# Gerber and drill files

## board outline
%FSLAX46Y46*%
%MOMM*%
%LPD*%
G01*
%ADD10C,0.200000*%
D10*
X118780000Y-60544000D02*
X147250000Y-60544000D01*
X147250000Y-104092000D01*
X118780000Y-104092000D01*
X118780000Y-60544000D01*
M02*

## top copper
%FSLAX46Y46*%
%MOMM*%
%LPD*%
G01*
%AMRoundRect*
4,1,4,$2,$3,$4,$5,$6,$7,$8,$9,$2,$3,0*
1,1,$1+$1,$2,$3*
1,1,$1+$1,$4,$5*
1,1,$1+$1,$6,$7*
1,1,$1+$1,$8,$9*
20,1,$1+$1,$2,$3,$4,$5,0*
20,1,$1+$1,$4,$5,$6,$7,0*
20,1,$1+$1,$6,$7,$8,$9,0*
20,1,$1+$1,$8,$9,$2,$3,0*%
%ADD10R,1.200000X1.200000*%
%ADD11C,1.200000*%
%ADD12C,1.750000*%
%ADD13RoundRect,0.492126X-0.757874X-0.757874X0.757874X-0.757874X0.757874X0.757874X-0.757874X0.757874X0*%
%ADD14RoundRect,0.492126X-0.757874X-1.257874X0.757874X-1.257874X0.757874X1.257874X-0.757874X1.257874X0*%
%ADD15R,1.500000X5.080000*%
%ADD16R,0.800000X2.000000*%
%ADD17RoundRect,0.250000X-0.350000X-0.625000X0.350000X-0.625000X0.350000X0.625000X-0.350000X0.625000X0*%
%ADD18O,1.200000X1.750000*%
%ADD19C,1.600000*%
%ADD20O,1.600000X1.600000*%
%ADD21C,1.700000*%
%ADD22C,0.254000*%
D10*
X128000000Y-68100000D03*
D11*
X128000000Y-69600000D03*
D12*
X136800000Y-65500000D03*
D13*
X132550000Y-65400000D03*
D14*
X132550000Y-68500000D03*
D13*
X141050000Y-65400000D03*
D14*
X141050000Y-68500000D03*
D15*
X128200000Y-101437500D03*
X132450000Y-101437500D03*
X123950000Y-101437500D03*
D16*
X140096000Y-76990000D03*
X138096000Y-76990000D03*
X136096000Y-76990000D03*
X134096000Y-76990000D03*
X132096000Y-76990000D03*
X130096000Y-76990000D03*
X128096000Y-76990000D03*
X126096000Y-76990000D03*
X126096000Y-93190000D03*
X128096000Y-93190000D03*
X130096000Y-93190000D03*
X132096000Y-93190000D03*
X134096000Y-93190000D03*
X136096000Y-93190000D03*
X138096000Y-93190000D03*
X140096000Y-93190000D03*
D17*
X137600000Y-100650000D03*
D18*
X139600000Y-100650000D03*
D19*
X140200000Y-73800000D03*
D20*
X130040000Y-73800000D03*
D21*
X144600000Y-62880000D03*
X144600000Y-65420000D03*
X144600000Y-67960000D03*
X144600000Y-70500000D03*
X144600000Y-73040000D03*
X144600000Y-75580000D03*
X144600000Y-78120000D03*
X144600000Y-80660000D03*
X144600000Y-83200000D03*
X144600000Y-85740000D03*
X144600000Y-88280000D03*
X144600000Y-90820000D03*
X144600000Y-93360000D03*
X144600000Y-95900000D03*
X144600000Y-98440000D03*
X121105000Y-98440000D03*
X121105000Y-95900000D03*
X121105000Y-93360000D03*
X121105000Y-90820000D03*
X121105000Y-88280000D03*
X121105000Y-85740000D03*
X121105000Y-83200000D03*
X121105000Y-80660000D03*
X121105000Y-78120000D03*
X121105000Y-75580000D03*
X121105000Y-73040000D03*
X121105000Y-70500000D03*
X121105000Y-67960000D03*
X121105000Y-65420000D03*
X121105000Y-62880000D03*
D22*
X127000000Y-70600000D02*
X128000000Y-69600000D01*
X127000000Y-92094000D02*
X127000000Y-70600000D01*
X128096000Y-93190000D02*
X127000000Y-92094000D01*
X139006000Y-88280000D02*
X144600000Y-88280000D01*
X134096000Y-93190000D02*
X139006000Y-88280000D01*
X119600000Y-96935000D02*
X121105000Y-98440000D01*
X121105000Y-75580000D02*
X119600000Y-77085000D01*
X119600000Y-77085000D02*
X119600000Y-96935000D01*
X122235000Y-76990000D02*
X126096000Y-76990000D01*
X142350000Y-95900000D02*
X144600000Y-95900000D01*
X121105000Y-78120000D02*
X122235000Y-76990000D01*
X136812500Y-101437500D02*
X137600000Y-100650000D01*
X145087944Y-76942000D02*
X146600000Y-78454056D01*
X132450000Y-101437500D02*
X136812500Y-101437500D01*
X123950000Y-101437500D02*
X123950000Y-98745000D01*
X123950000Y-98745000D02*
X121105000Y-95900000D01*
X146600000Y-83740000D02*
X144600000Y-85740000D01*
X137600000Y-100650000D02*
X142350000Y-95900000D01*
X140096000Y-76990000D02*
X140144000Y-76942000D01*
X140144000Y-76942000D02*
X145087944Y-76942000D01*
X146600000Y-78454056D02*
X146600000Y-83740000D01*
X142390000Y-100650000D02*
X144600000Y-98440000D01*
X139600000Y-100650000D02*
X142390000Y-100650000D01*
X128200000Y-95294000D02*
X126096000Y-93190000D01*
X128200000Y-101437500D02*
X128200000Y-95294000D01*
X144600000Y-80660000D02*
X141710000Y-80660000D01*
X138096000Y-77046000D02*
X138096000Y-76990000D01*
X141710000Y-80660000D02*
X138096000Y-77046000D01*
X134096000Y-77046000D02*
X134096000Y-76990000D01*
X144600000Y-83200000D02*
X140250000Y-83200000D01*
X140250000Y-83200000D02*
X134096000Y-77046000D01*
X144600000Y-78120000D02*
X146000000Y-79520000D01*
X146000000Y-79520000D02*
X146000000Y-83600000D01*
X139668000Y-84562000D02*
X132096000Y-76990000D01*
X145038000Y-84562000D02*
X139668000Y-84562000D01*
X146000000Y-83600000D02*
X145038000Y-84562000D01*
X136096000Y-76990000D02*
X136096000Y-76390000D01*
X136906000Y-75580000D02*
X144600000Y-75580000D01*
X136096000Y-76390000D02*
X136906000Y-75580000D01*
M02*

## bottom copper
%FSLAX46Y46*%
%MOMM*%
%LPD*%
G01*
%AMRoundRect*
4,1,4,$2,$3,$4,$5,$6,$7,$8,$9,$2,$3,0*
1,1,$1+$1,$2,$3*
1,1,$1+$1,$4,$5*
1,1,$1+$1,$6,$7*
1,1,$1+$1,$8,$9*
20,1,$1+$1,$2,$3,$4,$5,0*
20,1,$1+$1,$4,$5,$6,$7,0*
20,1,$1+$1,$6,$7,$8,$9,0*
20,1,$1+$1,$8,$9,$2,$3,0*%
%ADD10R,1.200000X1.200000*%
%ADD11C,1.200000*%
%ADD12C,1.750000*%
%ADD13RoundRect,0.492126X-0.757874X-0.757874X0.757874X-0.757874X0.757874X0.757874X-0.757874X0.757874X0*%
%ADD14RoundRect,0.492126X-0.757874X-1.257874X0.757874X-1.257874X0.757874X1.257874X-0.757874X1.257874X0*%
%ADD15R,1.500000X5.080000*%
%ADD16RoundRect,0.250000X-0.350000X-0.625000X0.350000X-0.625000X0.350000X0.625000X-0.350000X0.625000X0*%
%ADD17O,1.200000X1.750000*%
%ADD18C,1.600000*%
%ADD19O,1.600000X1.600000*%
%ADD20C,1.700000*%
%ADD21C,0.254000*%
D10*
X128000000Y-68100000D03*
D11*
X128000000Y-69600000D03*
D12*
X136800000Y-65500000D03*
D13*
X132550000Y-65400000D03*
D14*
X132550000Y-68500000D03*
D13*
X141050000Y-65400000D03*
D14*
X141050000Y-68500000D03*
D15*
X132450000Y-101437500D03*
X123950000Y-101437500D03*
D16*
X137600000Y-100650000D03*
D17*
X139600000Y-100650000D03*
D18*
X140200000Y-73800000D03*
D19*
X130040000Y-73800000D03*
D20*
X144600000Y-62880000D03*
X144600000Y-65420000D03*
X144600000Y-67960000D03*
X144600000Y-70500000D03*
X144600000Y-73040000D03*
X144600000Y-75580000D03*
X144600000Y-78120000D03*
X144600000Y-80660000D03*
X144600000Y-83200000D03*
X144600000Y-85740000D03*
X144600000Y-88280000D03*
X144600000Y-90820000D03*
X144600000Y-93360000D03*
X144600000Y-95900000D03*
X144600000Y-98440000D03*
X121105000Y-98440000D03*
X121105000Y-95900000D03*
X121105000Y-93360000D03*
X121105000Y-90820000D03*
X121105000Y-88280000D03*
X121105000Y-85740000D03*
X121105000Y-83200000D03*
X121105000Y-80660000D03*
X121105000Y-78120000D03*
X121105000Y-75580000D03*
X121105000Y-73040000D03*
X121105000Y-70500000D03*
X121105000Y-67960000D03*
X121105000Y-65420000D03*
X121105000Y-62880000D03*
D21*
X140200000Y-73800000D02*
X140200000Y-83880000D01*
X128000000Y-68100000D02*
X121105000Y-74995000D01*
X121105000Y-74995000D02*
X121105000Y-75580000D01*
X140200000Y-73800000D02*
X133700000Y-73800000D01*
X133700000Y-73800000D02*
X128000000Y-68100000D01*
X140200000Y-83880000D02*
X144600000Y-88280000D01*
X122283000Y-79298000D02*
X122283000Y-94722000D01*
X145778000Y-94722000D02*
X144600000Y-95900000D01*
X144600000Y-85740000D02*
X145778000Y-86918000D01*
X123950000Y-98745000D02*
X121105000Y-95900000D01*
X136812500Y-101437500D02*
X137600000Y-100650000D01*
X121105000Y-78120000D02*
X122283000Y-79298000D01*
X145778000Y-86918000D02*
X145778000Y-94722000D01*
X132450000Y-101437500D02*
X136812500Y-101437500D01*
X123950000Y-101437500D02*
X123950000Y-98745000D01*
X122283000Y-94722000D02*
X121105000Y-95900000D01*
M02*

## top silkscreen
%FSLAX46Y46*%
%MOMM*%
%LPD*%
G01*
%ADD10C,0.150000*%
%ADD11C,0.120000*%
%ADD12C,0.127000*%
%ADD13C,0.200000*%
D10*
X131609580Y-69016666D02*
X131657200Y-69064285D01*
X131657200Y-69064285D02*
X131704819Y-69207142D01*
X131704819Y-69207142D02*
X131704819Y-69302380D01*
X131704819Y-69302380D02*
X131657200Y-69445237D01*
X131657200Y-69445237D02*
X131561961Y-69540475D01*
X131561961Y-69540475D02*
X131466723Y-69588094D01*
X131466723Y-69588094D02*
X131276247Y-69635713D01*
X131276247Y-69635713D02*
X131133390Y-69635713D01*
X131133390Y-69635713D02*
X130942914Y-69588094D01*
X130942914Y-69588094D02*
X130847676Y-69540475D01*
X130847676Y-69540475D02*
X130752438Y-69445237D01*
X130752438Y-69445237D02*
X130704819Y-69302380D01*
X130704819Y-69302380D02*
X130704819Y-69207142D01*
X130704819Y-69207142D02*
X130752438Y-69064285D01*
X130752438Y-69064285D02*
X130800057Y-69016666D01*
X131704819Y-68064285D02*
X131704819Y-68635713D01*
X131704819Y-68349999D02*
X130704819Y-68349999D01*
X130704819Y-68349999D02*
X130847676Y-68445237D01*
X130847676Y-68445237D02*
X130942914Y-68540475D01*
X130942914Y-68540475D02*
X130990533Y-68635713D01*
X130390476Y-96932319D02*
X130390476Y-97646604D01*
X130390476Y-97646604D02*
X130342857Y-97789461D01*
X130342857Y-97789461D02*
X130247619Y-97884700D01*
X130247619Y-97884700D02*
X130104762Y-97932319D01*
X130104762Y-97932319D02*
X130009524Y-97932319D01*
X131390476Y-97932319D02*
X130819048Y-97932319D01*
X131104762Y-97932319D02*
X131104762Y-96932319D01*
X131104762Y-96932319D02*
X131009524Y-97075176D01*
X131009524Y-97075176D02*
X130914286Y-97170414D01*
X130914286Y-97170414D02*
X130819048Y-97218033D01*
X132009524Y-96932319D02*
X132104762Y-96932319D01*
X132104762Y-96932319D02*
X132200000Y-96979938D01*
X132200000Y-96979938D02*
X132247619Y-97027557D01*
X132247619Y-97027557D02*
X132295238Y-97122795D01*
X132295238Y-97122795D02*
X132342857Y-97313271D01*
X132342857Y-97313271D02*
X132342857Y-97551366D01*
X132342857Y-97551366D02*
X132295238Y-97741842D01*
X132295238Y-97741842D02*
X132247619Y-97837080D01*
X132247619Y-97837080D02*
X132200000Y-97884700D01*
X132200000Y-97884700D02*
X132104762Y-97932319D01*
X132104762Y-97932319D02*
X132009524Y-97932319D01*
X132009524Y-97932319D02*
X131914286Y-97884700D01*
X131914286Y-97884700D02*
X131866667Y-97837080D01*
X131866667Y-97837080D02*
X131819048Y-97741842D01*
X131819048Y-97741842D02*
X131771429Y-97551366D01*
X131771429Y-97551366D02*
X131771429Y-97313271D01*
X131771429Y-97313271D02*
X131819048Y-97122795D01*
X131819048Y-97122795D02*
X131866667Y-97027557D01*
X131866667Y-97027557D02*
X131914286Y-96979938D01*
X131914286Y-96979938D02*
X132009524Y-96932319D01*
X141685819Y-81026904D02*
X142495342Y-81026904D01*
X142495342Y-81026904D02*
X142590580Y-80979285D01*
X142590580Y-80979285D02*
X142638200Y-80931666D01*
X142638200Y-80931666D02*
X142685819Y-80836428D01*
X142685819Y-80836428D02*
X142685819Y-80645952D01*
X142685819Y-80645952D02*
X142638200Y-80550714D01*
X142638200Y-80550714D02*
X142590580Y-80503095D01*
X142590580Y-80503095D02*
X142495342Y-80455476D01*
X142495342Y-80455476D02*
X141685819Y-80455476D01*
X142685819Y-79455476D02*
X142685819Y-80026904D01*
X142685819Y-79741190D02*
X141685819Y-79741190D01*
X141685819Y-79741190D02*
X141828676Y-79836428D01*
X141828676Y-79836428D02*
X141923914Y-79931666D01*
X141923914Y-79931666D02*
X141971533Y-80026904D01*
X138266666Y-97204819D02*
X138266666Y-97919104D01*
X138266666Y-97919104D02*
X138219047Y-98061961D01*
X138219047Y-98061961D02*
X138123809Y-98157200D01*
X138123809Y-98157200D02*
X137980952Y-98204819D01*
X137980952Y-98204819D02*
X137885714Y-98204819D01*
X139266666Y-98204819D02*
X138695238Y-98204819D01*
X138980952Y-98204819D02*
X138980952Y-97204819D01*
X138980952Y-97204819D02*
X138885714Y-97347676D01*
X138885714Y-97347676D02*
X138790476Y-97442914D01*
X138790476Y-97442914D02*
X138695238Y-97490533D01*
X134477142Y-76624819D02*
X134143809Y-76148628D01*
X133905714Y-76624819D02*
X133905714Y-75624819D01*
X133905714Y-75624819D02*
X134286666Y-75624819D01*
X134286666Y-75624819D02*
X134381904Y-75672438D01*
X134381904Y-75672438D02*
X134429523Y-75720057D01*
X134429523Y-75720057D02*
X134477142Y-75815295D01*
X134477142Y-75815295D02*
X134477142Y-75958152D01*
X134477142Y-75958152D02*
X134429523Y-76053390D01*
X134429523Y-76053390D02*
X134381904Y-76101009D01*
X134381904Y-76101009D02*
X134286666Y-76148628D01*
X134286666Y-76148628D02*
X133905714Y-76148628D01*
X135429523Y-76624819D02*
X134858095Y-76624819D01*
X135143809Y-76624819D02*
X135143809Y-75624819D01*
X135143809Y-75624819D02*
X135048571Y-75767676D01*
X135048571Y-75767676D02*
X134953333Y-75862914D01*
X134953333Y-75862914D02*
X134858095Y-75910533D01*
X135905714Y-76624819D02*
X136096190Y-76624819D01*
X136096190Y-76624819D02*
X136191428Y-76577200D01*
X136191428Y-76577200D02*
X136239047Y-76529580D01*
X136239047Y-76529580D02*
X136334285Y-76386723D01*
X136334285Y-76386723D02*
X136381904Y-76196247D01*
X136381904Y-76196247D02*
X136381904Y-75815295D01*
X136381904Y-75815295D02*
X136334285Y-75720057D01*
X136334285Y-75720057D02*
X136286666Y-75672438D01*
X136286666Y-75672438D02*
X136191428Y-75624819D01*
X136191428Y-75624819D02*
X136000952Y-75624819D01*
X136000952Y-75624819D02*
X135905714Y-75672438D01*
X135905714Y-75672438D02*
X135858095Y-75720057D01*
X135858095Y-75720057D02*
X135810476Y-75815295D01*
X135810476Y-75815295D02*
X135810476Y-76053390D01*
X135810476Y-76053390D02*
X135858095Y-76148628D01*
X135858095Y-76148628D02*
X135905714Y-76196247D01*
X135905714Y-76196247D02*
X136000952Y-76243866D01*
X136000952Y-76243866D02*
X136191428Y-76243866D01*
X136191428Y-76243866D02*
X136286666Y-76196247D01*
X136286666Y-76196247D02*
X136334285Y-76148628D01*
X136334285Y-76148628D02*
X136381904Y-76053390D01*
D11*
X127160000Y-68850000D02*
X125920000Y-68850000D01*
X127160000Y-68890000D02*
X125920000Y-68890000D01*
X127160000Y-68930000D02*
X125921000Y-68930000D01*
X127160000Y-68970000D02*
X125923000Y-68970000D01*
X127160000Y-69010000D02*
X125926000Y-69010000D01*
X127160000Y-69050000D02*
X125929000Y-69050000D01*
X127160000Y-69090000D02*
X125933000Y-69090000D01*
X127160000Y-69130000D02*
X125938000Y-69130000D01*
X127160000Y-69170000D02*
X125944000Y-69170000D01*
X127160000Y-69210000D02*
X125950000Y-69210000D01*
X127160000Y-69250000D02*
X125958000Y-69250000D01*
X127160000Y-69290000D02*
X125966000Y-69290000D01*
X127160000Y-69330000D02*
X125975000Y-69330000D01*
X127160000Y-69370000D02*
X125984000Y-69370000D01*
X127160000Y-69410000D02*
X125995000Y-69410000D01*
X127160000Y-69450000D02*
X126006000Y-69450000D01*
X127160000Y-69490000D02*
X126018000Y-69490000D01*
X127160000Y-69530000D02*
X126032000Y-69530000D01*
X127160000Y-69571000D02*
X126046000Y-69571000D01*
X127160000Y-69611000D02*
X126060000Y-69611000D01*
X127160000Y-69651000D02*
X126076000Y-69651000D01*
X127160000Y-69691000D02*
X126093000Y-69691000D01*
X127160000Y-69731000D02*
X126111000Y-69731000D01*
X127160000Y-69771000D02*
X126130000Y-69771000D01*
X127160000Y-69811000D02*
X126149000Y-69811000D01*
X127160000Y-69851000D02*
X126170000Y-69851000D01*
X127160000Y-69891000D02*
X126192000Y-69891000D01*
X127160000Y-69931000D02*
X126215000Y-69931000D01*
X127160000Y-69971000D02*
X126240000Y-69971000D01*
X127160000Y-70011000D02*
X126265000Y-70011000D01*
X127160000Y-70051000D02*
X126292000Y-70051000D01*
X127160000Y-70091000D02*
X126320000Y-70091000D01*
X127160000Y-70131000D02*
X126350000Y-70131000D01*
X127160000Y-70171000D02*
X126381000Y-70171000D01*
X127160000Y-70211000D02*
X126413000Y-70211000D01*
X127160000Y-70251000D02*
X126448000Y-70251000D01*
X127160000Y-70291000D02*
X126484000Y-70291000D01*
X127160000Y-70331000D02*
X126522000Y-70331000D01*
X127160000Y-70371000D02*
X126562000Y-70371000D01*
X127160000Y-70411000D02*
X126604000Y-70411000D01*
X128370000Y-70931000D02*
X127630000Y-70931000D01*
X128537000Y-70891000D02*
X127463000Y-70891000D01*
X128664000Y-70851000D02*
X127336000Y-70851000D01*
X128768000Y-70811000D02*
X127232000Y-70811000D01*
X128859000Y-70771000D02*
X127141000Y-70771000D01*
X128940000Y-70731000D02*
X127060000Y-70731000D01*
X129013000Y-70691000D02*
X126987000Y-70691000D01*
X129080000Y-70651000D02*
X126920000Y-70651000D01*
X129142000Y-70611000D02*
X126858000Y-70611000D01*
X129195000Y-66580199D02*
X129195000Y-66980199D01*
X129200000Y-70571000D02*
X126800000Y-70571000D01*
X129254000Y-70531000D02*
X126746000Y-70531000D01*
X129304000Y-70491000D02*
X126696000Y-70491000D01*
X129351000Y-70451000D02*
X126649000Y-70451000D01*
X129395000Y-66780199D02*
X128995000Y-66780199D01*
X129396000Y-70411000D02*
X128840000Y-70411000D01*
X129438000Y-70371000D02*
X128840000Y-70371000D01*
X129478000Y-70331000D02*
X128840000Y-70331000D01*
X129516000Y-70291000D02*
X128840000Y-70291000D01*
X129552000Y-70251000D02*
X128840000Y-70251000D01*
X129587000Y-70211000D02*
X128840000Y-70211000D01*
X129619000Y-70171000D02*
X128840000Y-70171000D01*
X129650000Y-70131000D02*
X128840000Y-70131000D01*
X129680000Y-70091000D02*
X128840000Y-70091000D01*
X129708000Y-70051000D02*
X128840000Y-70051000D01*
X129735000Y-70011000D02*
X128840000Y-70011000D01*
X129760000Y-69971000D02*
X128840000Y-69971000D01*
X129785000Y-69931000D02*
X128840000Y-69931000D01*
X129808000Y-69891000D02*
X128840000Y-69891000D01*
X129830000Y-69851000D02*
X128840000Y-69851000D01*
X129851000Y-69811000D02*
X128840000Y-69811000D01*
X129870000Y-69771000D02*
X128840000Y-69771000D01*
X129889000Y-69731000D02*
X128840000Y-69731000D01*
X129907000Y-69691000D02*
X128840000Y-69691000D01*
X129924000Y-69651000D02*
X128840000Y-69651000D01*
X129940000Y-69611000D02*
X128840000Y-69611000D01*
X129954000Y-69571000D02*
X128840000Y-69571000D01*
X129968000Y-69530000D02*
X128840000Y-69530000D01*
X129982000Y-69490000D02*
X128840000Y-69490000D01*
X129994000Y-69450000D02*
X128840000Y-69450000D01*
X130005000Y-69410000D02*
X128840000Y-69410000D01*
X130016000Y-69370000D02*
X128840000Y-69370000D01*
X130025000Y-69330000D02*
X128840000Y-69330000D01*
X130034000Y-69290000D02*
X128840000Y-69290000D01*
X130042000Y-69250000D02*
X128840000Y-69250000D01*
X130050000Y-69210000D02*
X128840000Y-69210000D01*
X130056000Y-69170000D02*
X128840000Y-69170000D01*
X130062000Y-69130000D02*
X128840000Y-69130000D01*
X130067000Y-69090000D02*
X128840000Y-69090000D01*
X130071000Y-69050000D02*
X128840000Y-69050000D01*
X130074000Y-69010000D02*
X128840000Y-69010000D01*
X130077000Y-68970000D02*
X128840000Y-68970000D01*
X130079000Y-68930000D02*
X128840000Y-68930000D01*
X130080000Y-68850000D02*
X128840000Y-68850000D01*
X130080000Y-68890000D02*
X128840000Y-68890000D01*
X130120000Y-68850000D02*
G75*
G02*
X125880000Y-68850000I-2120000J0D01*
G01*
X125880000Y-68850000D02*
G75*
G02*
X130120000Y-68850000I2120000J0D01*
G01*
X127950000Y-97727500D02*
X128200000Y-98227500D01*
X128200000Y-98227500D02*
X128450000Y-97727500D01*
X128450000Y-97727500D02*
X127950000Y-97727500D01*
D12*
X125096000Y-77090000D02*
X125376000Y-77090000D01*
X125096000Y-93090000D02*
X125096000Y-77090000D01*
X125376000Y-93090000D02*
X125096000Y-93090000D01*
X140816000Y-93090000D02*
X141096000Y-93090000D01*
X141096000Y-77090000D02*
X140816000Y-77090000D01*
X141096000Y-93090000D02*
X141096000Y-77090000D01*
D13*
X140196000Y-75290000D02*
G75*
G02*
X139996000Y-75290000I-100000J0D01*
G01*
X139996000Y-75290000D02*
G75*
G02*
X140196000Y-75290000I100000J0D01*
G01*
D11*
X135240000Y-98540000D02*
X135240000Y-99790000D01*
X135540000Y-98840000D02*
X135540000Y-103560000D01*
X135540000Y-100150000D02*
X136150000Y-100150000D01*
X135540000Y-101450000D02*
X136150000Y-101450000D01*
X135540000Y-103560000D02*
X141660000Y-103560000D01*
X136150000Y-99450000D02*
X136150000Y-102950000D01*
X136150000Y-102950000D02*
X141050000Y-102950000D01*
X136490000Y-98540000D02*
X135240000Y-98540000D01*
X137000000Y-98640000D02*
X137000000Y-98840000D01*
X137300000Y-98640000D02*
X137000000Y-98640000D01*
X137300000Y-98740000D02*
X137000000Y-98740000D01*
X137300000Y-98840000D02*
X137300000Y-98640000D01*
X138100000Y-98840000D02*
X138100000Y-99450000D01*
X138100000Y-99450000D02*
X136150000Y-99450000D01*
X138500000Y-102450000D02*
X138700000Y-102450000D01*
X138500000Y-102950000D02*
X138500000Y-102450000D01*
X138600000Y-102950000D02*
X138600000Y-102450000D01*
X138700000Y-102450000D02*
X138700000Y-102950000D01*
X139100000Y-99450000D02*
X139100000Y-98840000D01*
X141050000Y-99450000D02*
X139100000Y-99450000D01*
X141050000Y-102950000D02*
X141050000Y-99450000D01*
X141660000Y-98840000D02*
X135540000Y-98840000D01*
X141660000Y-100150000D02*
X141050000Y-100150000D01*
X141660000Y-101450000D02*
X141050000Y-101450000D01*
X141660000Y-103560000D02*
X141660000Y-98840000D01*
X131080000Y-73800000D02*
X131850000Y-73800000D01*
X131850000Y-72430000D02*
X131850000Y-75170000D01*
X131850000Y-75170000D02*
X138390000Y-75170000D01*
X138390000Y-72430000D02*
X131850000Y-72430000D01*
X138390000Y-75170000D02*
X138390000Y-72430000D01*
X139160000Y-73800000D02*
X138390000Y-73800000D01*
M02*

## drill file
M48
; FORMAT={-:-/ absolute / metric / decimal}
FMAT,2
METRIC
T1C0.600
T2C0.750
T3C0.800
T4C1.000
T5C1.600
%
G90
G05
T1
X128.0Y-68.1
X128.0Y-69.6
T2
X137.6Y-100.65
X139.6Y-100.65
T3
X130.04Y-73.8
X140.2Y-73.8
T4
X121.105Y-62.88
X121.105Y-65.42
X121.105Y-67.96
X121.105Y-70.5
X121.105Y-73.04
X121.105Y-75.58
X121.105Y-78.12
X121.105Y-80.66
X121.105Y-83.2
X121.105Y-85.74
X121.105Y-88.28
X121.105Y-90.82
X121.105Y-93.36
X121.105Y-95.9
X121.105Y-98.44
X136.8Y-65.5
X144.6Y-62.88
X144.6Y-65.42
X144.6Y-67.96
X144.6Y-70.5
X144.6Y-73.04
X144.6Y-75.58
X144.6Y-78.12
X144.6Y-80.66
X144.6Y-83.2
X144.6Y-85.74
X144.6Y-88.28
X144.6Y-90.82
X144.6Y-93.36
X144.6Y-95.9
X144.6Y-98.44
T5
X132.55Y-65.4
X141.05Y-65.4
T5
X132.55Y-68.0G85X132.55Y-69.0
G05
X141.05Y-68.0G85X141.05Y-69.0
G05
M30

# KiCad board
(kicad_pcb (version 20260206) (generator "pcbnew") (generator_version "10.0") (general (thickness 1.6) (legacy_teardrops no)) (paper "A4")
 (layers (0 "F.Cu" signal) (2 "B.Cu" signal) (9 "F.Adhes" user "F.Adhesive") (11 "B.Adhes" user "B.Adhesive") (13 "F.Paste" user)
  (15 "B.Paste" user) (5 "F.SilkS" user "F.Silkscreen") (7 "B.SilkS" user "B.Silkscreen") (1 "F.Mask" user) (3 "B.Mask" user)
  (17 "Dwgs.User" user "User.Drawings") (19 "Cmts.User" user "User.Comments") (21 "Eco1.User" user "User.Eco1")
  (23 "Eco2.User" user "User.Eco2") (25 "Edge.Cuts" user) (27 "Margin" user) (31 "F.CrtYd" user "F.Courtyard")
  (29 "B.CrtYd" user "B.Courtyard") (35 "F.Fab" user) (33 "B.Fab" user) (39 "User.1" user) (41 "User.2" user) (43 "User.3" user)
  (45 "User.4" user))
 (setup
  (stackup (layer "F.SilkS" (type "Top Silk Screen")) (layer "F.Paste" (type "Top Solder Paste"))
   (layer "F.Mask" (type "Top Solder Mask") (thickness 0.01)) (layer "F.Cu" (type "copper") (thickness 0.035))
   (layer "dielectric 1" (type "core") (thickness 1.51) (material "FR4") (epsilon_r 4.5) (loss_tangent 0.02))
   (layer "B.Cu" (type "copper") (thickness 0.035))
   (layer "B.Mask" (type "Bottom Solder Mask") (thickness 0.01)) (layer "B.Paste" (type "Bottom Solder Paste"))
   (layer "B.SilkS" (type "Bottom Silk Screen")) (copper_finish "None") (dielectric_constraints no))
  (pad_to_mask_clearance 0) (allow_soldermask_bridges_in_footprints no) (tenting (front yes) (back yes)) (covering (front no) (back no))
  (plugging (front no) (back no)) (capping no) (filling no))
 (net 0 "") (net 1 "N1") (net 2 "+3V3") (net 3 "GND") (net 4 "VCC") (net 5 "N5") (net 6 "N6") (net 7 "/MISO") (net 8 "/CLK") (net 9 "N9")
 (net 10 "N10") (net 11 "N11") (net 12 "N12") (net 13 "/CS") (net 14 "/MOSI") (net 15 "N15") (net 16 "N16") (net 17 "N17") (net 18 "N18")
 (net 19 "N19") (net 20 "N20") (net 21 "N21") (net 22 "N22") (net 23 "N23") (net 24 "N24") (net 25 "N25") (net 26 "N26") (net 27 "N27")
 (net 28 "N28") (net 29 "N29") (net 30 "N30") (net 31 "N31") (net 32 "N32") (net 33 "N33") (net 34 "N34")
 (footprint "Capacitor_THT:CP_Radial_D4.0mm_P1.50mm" (layer "F.Cu") (at 128 68.1 -90)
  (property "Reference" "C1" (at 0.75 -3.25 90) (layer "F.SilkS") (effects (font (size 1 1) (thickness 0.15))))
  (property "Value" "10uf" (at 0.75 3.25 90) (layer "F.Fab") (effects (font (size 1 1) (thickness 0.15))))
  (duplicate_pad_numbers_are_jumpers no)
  (fp_line (start 0.75 0.84) (end 0.75 2.08) (stroke (width 0.12) (type solid)) (layer "F.SilkS"))
  (fp_line (start 0.79 0.84) (end 0.79 2.08) (stroke (width 0.12) (type solid)) (layer "F.SilkS"))
  (fp_line (start 0.83 0.84) (end 0.83 2.079) (stroke (width 0.12) (type solid)) (layer "F.SilkS"))
  (fp_line (start 0.87 0.84) (end 0.87 2.077) (stroke (width 0.12) (type solid)) (layer "F.SilkS"))
  (fp_line (start 0.91 0.84) (end 0.91 2.074) (stroke (width 0.12) (type solid)) (layer "F.SilkS"))
  (fp_line (start 0.95 0.84) (end 0.95 2.071) (stroke (width 0.12) (type solid)) (layer "F.SilkS"))
  (fp_line (start 0.99 0.84) (end 0.99 2.067) (stroke (width 0.12) (type solid)) (layer "F.SilkS"))
  (fp_line (start 1.03 0.84) (end 1.03 2.062) (stroke (width 0.12) (type solid)) (layer "F.SilkS"))
  (fp_line (start 1.07 0.84) (end 1.07 2.056) (stroke (width 0.12) (type solid)) (layer "F.SilkS"))
  (fp_line (start 1.11 0.84) (end 1.11 2.05) (stroke (width 0.12) (type solid)) (layer "F.SilkS"))
  (fp_line (start 1.15 0.84) (end 1.15 2.042) (stroke (width 0.12) (type solid)) (layer "F.SilkS"))
  (fp_line (start 1.19 0.84) (end 1.19 2.034) (stroke (width 0.12) (type solid)) (layer "F.SilkS"))
  (fp_line (start 1.23 0.84) (end 1.23 2.025) (stroke (width 0.12) (type solid)) (layer "F.SilkS"))
  (fp_line (start 1.27 0.84) (end 1.27 2.016) (stroke (width 0.12) (type solid)) (layer "F.SilkS"))
  (fp_line (start 1.31 0.84) (end 1.31 2.005) (stroke (width 0.12) (type solid)) (layer "F.SilkS"))
  (fp_line (start 1.35 0.84) (end 1.35 1.994) (stroke (width 0.12) (type solid)) (layer "F.SilkS"))
  (fp_line (start 1.39 0.84) (end 1.39 1.982) (stroke (width 0.12) (type solid)) (layer "F.SilkS"))
  (fp_line (start 1.43 0.84) (end 1.43 1.968) (stroke (width 0.12) (type solid)) (layer "F.SilkS"))
  (fp_line (start 1.471 0.84) (end 1.471 1.954) (stroke (width 0.12) (type solid)) (layer "F.SilkS"))
  (fp_line (start 1.511 0.84) (end 1.511 1.94) (stroke (width 0.12) (type solid)) (layer "F.SilkS"))
  (fp_line (start 1.551 0.84) (end 1.551 1.924) (stroke (width 0.12) (type solid)) (layer "F.SilkS"))
  (fp_line (start 1.591 0.84) (end 1.591 1.907) (stroke (width 0.12) (type solid)) (layer "F.SilkS"))
  (fp_line (start 1.631 0.84) (end 1.631 1.889) (stroke (width 0.12) (type solid)) (layer "F.SilkS"))
  (fp_line (start 1.671 0.84) (end 1.671 1.87) (stroke (width 0.12) (type solid)) (layer "F.SilkS"))
  (fp_line (start 1.711 0.84) (end 1.711 1.851) (stroke (width 0.12) (type solid)) (layer "F.SilkS"))
  (fp_line (start 1.751 0.84) (end 1.751 1.83) (stroke (width 0.12) (type solid)) (layer "F.SilkS"))
  (fp_line (start 1.791 0.84) (end 1.791 1.808) (stroke (width 0.12) (type solid)) (layer "F.SilkS"))
  (fp_line (start 1.831 0.84) (end 1.831 1.785) (stroke (width 0.12) (type solid)) (layer "F.SilkS"))
  (fp_line (start 1.871 0.84) (end 1.871 1.76) (stroke (width 0.12) (type solid)) (layer "F.SilkS"))
  (fp_line (start 1.911 0.84) (end 1.911 1.735) (stroke (width 0.12) (type solid)) (layer "F.SilkS"))
  (fp_line (start 1.951 0.84) (end 1.951 1.708) (stroke (width 0.12) (type solid)) (layer "F.SilkS"))
  (fp_line (start 1.991 0.84) (end 1.991 1.68) (stroke (width 0.12) (type solid)) (layer "F.SilkS"))
  (fp_line (start 2.031 0.84) (end 2.031 1.65) (stroke (width 0.12) (type solid)) (layer "F.SilkS"))
  (fp_line (start 2.071 0.84) (end 2.071 1.619) (stroke (width 0.12) (type solid)) (layer "F.SilkS"))
  (fp_line (start 2.111 0.84) (end 2.111 1.587) (stroke (width 0.12) (type solid)) (layer "F.SilkS"))
  (fp_line (start 2.151 0.84) (end 2.151 1.552) (stroke (width 0.12) (type solid)) (layer "F.SilkS"))
  (fp_line (start 2.191 0.84) (end 2.191 1.516) (stroke (width 0.12) (type solid)) (layer "F.SilkS"))
  (fp_line (start 2.231 0.84) (end 2.231 1.478) (stroke (width 0.12) (type solid)) (layer "F.SilkS"))
  (fp_line (start 2.271 0.84) (end 2.271 1.438) (stroke (width 0.12) (type solid)) (layer "F.SilkS"))
  (fp_line (start 2.311 0.84) (end 2.311 1.396) (stroke (width 0.12) (type solid)) (layer "F.SilkS"))
  (fp_line (start 2.831 -0.37) (end 2.831 0.37) (stroke (width 0.12) (type solid)) (layer "F.SilkS"))
  (fp_line (start 2.791 -0.537) (end 2.791 0.537) (stroke (width 0.12) (type solid)) (layer "F.SilkS"))
  (fp_line (start 2.751 -0.664) (end 2.751 0.664) (stroke (width 0.12) (type solid)) (layer "F.SilkS"))
  (fp_line (start 2.711 -0.768) (end 2.711 0.768) (stroke (width 0.12) (type solid)) (layer "F.SilkS"))
  (fp_line (start 2.671 -0.859) (end 2.671 0.859) (stroke (width 0.12) (type solid)) (layer "F.SilkS"))
  (fp_line (start 2.631 -0.94) (end 2.631 0.94) (stroke (width 0.12) (type solid)) (layer "F.SilkS"))
  (fp_line (start 2.591 -1.013) (end 2.591 1.013) (stroke (width 0.12) (type solid)) (layer "F.SilkS"))
  (fp_line (start 2.551 -1.08) (end 2.551 1.08) (stroke (width 0.12) (type solid)) (layer "F.SilkS"))
  (fp_line (start 2.511 -1.142) (end 2.511 1.142) (stroke (width 0.12) (type solid)) (layer "F.SilkS"))
  (fp_line (start -1.519801 -1.195) (end -1.119801 -1.195) (stroke (width 0.12) (type solid)) (layer "F.SilkS"))
  (fp_line (start 2.471 -1.2) (end 2.471 1.2) (stroke (width 0.12) (type solid)) (layer "F.SilkS"))
  (fp_line (start 2.431 -1.254) (end 2.431 1.254) (stroke (width 0.12) (type solid)) (layer "F.SilkS"))
  (fp_line (start 2.391 -1.304) (end 2.391 1.304) (stroke (width 0.12) (type solid)) (layer "F.SilkS"))
  (fp_line (start 2.351 -1.351) (end 2.351 1.351) (stroke (width 0.12) (type solid)) (layer "F.SilkS"))
  (fp_line (start -1.319801 -1.395) (end -1.319801 -0.995) (stroke (width 0.12) (type solid)) (layer "F.SilkS"))
  (fp_line (start 2.311 -1.396) (end 2.311 -0.84) (stroke (width 0.12) (type solid)) (layer "F.SilkS"))
  (fp_line (start 2.271 -1.438) (end 2.271 -0.84) (stroke (width 0.12) (type solid)) (layer "F.SilkS"))
  (fp_line (start 2.231 -1.478) (end 2.231 -0.84) (stroke (width 0.12) (type solid)) (layer "F.SilkS"))
  (fp_line (start 2.191 -1.516) (end 2.191 -0.84) (stroke (width 0.12) (type solid)) (layer "F.SilkS"))
  (fp_line (start 2.151 -1.552) (end 2.151 -0.84) (stroke (width 0.12) (type solid)) (layer "F.SilkS"))
  (fp_line (start 2.111 -1.587) (end 2.111 -0.84) (stroke (width 0.12) (type solid)) (layer "F.SilkS"))
  (fp_line (start 2.071 -1.619) (end 2.071 -0.84) (stroke (width 0.12) (type solid)) (layer "F.SilkS"))
  (fp_line (start 2.031 -1.65) (end 2.031 -0.84) (stroke (width 0.12) (type solid)) (layer "F.SilkS"))
  (fp_line (start 1.991 -1.68) (end 1.991 -0.84) (stroke (width 0.12) (type solid)) (layer "F.SilkS"))
  (fp_line (start 1.951 -1.708) (end 1.951 -0.84) (stroke (width 0.12) (type solid)) (layer "F.SilkS"))
  (fp_line (start 1.911 -1.735) (end 1.911 -0.84) (stroke (width 0.12) (type solid)) (layer "F.SilkS"))
  (fp_line (start 1.871 -1.76) (end 1.871 -0.84) (stroke (width 0.12) (type solid)) (layer "F.SilkS"))
  (fp_line (start 1.831 -1.785) (end 1.831 -0.84) (stroke (width 0.12) (type solid)) (layer "F.SilkS"))
  (fp_line (start 1.791 -1.808) (end 1.791 -0.84) (stroke (width 0.12) (type solid)) (layer "F.SilkS"))
  (fp_line (start 1.751 -1.83) (end 1.751 -0.84) (stroke (width 0.12) (type solid)) (layer "F.SilkS"))
  (fp_line (start 1.711 -1.851) (end 1.711 -0.84) (stroke (width 0.12) (type solid)) (layer "F.SilkS"))
  (fp_line (start 1.671 -1.87) (end 1.671 -0.84) (stroke (width 0.12) (type solid)) (layer "F.SilkS"))
  (fp_line (start 1.631 -1.889) (end 1.631 -0.84) (stroke (width 0.12) (type solid)) (layer "F.SilkS"))
  (fp_line (start 1.591 -1.907) (end 1.591 -0.84) (stroke (width 0.12) (type solid)) (layer "F.SilkS"))
  (fp_line (start 1.551 -1.924) (end 1.551 -0.84) (stroke (width 0.12) (type solid)) (layer "F.SilkS"))
  (fp_line (start 1.511 -1.94) (end 1.511 -0.84) (stroke (width 0.12) (type solid)) (layer "F.SilkS"))
  (fp_line (start 1.471 -1.954) (end 1.471 -0.84) (stroke (width 0.12) (type solid)) (layer "F.SilkS"))
  (fp_line (start 1.43 -1.968) (end 1.43 -0.84) (stroke (width 0.12) (type solid)) (layer "F.SilkS"))
  (fp_line (start 1.39 -1.982) (end 1.39 -0.84) (stroke (width 0.12) (type solid)) (layer "F.SilkS"))
  (fp_line (start 1.35 -1.994) (end 1.35 -0.84) (stroke (width 0.12) (type solid)) (layer "F.SilkS"))
  (fp_line (start 1.31 -2.005) (end 1.31 -0.84) (stroke (width 0.12) (type solid)) (layer "F.SilkS"))
  (fp_line (start 1.27 -2.016) (end 1.27 -0.84) (stroke (width 0.12) (type solid)) (layer "F.SilkS"))
  (fp_line (start 1.23 -2.025) (end 1.23 -0.84) (stroke (width 0.12) (type solid)) (layer "F.SilkS"))
  (fp_line (start 1.19 -2.034) (end 1.19 -0.84) (stroke (width 0.12) (type solid)) (layer "F.SilkS"))
  (fp_line (start 1.15 -2.042) (end 1.15 -0.84) (stroke (width 0.12) (type solid)) (layer "F.SilkS"))
  (fp_line (start 1.11 -2.05) (end 1.11 -0.84) (stroke (width 0.12) (type solid)) (layer "F.SilkS"))
  (fp_line (start 1.07 -2.056) (end 1.07 -0.84) (stroke (width 0.12) (type solid)) (layer "F.SilkS"))
  (fp_line (start 1.03 -2.062) (end 1.03 -0.84) (stroke (width 0.12) (type solid)) (layer "F.SilkS"))
  (fp_line (start 0.99 -2.067) (end 0.99 -0.84) (stroke (width 0.12) (type solid)) (layer "F.SilkS"))
  (fp_line (start 0.95 -2.071) (end 0.95 -0.84) (stroke (width 0.12) (type solid)) (layer "F.SilkS"))
  (fp_line (start 0.91 -2.074) (end 0.91 -0.84) (stroke (width 0.12) (type solid)) (layer "F.SilkS"))
  (fp_line (start 0.87 -2.077) (end 0.87 -0.84) (stroke (width 0.12) (type solid)) (layer "F.SilkS"))
  (fp_line (start 0.83 -2.079) (end 0.83 -0.84) (stroke (width 0.12) (type solid)) (layer "F.SilkS"))
  (fp_line (start 0.75 -2.08) (end 0.75 -0.84) (stroke (width 0.12) (type solid)) (layer "F.SilkS"))
  (fp_line (start 0.79 -2.08) (end 0.79 -0.84) (stroke (width 0.12) (type solid)) (layer "F.SilkS"))
  (fp_circle (center 0.75 0) (end 2.87 0) (stroke (width 0.12) (type solid)) (fill no) (layer "F.SilkS"))
  (pad "1" thru_hole rect (at 0 0 270) (size 1.2 1.2) (drill 0.6) (layers "*.Cu" "*.Mask") (remove_unused_layers no) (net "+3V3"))
  (pad "2" thru_hole circle (at 1.5 0 270) (size 1.2 1.2) (drill 0.6) (layers "*.Cu" "*.Mask") (remove_unused_layers no) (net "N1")))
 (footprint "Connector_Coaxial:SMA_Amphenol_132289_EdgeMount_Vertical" (layer "F.Cu") (at 136.8 65.5)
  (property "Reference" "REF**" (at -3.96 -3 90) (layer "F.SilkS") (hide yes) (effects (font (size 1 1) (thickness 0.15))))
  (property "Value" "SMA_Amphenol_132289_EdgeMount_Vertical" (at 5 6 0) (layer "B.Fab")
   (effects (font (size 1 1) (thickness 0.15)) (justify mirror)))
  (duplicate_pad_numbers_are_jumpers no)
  (pad "1" thru_hole circle (at 0 0) (size 1.75 1.75) (drill 1) (layers "*.Cu" "*.Mask") (remove_unused_layers no))
  (pad "2" thru_hole roundrect (at -4.25 -0.1) (size 2.5 2.5) (drill 1.6) (layers "*.Cu" "*.Mask") (remove_unused_layers no)
   (roundrect_rratio 0.1968503937) (thermal_bridge_angle 45))
  (pad "2" thru_hole roundrect (at -4.25 3) (size 2.5 3.5) (drill oval 1.6 2.6) (layers "*.Cu" "*.Mask") (remove_unused_layers no)
   (roundrect_rratio 0.1968503937) (thermal_bridge_angle 45))
  (pad "2" thru_hole roundrect (at 4.25 -0.1) (size 2.5 2.5) (drill 1.6) (layers "*.Cu" "*.Mask") (remove_unused_layers no)
   (roundrect_rratio 0.1968503937) (thermal_bridge_angle 45))
  (pad "2" thru_hole roundrect (at 4.25 3) (size 2.5 3.5) (drill oval 1.6 2.6) (layers "*.Cu" "*.Mask") (remove_unused_layers no)
   (roundrect_rratio 0.1968503937) (thermal_bridge_angle 45)))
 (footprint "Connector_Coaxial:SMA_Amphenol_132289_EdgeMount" (layer "F.Cu") (at 128.2 101.4375 -90)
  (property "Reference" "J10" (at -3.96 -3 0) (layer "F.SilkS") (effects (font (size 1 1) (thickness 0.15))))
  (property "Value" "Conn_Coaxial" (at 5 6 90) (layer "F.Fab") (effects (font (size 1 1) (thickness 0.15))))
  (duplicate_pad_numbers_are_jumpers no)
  (fp_line (start -3.71 0.25) (end -3.21 0) (stroke (width 0.12) (type solid)) (layer "F.SilkS"))
  (fp_line (start -3.21 0) (end -3.71 -0.25) (stroke (width 0.12) (type solid)) (layer "F.SilkS"))
  (fp_line (start -3.71 -0.25) (end -3.71 0.25) (stroke (width 0.12) (type solid)) (layer "F.SilkS"))
  (pad "1" smd rect (at 0 0) (size 1.5 5.08) (layers "F.Cu" "F.Mask" "F.Paste") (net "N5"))
  (pad "2" smd rect (at 0 -4.25) (size 1.5 5.08) (layers "F.Cu" "F.Mask" "F.Paste") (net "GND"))
  (pad "2" smd rect (at 0 -4.25) (size 1.5 5.08) (layers "B.Cu" "B.Mask" "B.Paste") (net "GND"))
  (pad "2" smd rect (at 0 4.25) (size 1.5 5.08) (layers "F.Cu" "F.Mask" "F.Paste") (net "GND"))
  (pad "2" smd rect (at 0 4.25) (size 1.5 5.08) (layers "B.Cu" "B.Mask" "B.Paste") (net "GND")))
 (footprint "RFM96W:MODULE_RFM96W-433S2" (layer "F.Cu") (at 133.096 85.09 -90)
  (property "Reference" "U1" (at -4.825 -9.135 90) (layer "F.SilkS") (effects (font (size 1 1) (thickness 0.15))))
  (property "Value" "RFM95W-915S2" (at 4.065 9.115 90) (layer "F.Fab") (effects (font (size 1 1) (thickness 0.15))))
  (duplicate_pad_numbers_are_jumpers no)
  (fp_line (start -8 8) (end -8 7.72) (stroke (width 0.127) (type solid)) (layer "F.SilkS"))
  (fp_line (start 8 8) (end -8 8) (stroke (width 0.127) (type solid)) (layer "F.SilkS"))
  (fp_line (start 8 7.72) (end 8 8) (stroke (width 0.127) (type solid)) (layer "F.SilkS"))
  (fp_line (start 8 -7.72) (end 8 -8) (stroke (width 0.127) (type solid)) (layer "F.SilkS"))
  (fp_line (start -8 -8) (end -8 -7.72) (stroke (width 0.127) (type solid)) (layer "F.SilkS"))
  (fp_line (start 8 -8) (end -8 -8) (stroke (width 0.127) (type solid)) (layer "F.SilkS"))
  (fp_circle (center -9.8 -7) (end -9.7 -7) (stroke (width 0.2) (type solid)) (fill no) (layer "F.SilkS"))
  (pad "1" smd rect (at -8.1 -7 270) (size 2 0.8) (layers "F.Cu" "F.Mask" "F.Paste") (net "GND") (solder_mask_margin 0.102))
  (pad "2" smd rect (at -8.1 -5 270) (size 2 0.8) (layers "F.Cu" "F.Mask" "F.Paste") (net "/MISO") (solder_mask_margin 0.102))
  (pad "3" smd rect (at -8.1 -3 270) (size 2 0.8) (layers "F.Cu" "F.Mask" "F.Paste") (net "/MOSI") (solder_mask_margin 0.102))
  (pad "4" smd rect (at -8.1 -1 270) (size 2 0.8) (layers "F.Cu" "F.Mask" "F.Paste") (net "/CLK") (solder_mask_margin 0.102))
  (pad "5" smd rect (at -8.1 1 270) (size 2 0.8) (layers "F.Cu" "F.Mask" "F.Paste") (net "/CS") (solder_mask_margin 0.102))
  (pad "6" smd rect (at -8.1 3 270) (size 2 0.8) (layers "F.Cu" "F.Mask" "F.Paste") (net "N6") (solder_mask_margin 0.102))
  (pad "7" smd rect (at -8.1 5 270) (size 2 0.8) (layers "F.Cu" "F.Mask" "F.Paste") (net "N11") (solder_mask_margin 0.102))
  (pad "8" smd rect (at -8.1 7 270) (size 2 0.8) (layers "F.Cu" "F.Mask" "F.Paste") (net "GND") (solder_mask_margin 0.102))
  (pad "9" smd rect (at 8.1 7 270) (size 2 0.8) (layers "F.Cu" "F.Mask" "F.Paste") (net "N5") (solder_mask_margin 0.102))
  (pad "10" smd rect (at 8.1 5 270) (size 2 0.8) (layers "F.Cu" "F.Mask" "F.Paste") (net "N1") (solder_mask_margin 0.102))
  (pad "11" smd rect (at 8.1 3 270) (size 2 0.8) (layers "F.Cu" "F.Mask" "F.Paste") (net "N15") (solder_mask_margin 0.102))
  (pad "12" smd rect (at 8.1 1 270) (size 2 0.8) (layers "F.Cu" "F.Mask" "F.Paste") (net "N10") (solder_mask_margin 0.102))
  (pad "13" smd rect (at 8.1 -1 270) (size 2 0.8) (layers "F.Cu" "F.Mask" "F.Paste") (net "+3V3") (solder_mask_margin 0.102))
  (pad "14" smd rect (at 8.1 -3 270) (size 2 0.8) (layers "F.Cu" "F.Mask" "F.Paste") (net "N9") (solder_mask_margin 0.102))
  (pad "15" smd rect (at 8.1 -5 270) (size 2 0.8) (layers "F.Cu" "F.Mask" "F.Paste") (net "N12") (solder_mask_margin 0.102))
  (pad "16" smd rect (at 8.1 -7 270) (size 2 0.8) (layers "F.Cu" "F.Mask" "F.Paste") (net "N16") (solder_mask_margin 0.102)))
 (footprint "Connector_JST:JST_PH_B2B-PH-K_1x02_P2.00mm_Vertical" (layer "F.Cu") (at 137.6 100.65)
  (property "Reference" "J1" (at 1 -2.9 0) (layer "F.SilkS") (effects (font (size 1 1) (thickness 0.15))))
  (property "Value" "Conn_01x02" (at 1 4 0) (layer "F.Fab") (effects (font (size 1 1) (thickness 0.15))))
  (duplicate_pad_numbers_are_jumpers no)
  (fp_line (start -2.36 -2.11) (end -2.36 -0.86) (stroke (width 0.12) (type solid)) (layer "F.SilkS"))
  (fp_line (start -2.06 -1.81) (end -2.06 2.91) (stroke (width 0.12) (type solid)) (layer "F.SilkS"))
  (fp_line (start -2.06 -0.5) (end -1.45 -0.5) (stroke (width 0.12) (type solid)) (layer "F.SilkS"))
  (fp_line (start -2.06 0.8) (end -1.45 0.8) (stroke (width 0.12) (type solid)) (layer "F.SilkS"))
  (fp_line (start -2.06 2.91) (end 4.06 2.91) (stroke (width 0.12) (type solid)) (layer "F.SilkS"))
  (fp_line (start -1.45 -1.2) (end -1.45 2.3) (stroke (width 0.12) (type solid)) (layer "F.SilkS"))
  (fp_line (start -1.45 2.3) (end 3.45 2.3) (stroke (width 0.12) (type solid)) (layer "F.SilkS"))
  (fp_line (start -1.11 -2.11) (end -2.36 -2.11) (stroke (width 0.12) (type solid)) (layer "F.SilkS"))
  (fp_line (start -0.6 -2.01) (end -0.6 -1.81) (stroke (width 0.12) (type solid)) (layer "F.SilkS"))
  (fp_line (start -0.3 -2.01) (end -0.6 -2.01) (stroke (width 0.12) (type solid)) (layer "F.SilkS"))
  (fp_line (start -0.3 -1.91) (end -0.6 -1.91) (stroke (width 0.12) (type solid)) (layer "F.SilkS"))
  (fp_line (start -0.3 -1.81) (end -0.3 -2.01) (stroke (width 0.12) (type solid)) (layer "F.SilkS"))
  (fp_line (start 0.5 -1.81) (end 0.5 -1.2) (stroke (width 0.12) (type solid)) (layer "F.SilkS"))
  (fp_line (start 0.5 -1.2) (end -1.45 -1.2) (stroke (width 0.12) (type solid)) (layer "F.SilkS"))
  (fp_line (start 0.9 1.8) (end 1.1 1.8) (stroke (width 0.12) (type solid)) (layer "F.SilkS"))
  (fp_line (start 0.9 2.3) (end 0.9 1.8) (stroke (width 0.12) (type solid)) (layer "F.SilkS"))
  (fp_line (start 1 2.3) (end 1 1.8) (stroke (width 0.12) (type solid)) (layer "F.SilkS"))
  (fp_line (start 1.1 1.8) (end 1.1 2.3) (stroke (width 0.12) (type solid)) (layer "F.SilkS"))
  (fp_line (start 1.5 -1.2) (end 1.5 -1.81) (stroke (width 0.12) (type solid)) (layer "F.SilkS"))
  (fp_line (start 3.45 -1.2) (end 1.5 -1.2) (stroke (width 0.12) (type solid)) (layer "F.SilkS"))
  (fp_line (start 3.45 2.3) (end 3.45 -1.2) (stroke (width 0.12) (type solid)) (layer "F.SilkS"))
  (fp_line (start 4.06 -1.81) (end -2.06 -1.81) (stroke (width 0.12) (type solid)) (layer "F.SilkS"))
  (fp_line (start 4.06 -0.5) (end 3.45 -0.5) (stroke (width 0.12) (type solid)) (layer "F.SilkS"))
  (fp_line (start 4.06 0.8) (end 3.45 0.8) (stroke (width 0.12) (type solid)) (layer "F.SilkS"))
  (fp_line (start 4.06 2.91) (end 4.06 -1.81) (stroke (width 0.12) (type solid)) (layer "F.SilkS"))
  (pad "1" thru_hole roundrect (at 0 0) (size 1.2 1.75) (drill 0.75) (layers "*.Cu" "*.Mask") (remove_unused_layers no)
   (roundrect_rratio 0.208333) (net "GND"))
  (pad "2" thru_hole oval (at 2 0) (size 1.2 1.75) (drill 0.75) (layers "*.Cu" "*.Mask") (remove_unused_layers no) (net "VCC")))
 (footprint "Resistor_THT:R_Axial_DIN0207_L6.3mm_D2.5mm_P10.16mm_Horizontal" (layer "F.Cu") (at 140.2 73.8 180)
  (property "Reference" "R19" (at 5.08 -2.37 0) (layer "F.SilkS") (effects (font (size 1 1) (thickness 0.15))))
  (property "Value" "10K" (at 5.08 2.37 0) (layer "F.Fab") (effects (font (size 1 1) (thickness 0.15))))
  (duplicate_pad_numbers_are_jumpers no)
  (fp_line (start 9.12 0) (end 8.35 0) (stroke (width 0.12) (type solid)) (layer "F.SilkS"))
  (fp_line (start 8.35 1.37) (end 8.35 -1.37) (stroke (width 0.12) (type solid)) (layer "F.SilkS"))
  (fp_line (start 8.35 -1.37) (end 1.81 -1.37) (stroke (width 0.12) (type solid)) (layer "F.SilkS"))
  (fp_line (start 1.81 1.37) (end 8.35 1.37) (stroke (width 0.12) (type solid)) (layer "F.SilkS"))
  (fp_line (start 1.81 -1.37) (end 1.81 1.37) (stroke (width 0.12) (type solid)) (layer "F.SilkS"))
  (fp_line (start 1.04 0) (end 1.81 0) (stroke (width 0.12) (type solid)) (layer "F.SilkS"))
  (pad "1" thru_hole circle (at 0 0 180) (size 1.6 1.6) (drill 0.8) (layers "*.Cu" "*.Mask") (remove_unused_layers no) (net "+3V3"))
  (pad "2" thru_hole oval (at 10.16 0 180) (size 1.6 1.6) (drill 0.8) (layers "*.Cu" "*.Mask") (remove_unused_layers no) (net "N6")))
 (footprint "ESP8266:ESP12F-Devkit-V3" (layer "B.Cu") (at 132.535 81.93 180)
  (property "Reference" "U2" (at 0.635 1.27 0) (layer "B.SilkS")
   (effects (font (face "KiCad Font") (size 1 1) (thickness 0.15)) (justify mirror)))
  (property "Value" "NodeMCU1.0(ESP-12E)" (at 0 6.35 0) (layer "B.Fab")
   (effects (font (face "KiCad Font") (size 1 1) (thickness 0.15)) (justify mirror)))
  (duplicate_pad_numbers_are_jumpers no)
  (pad "1" thru_hole circle (at -12.065 19.05 180) (size 1.7 1.7) (drill 1) (layers "*.Cu" "*.Mask" "B.SilkS") (remove_unused_layers no)
   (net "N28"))
  (pad "2" thru_hole circle (at -12.065 16.51 180) (size 1.7 1.7) (drill 1) (layers "*.Cu" "*.Mask" "B.SilkS") (remove_unused_layers no)
   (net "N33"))
  (pad "3" thru_hole circle (at -12.065 13.97 180) (size 1.7 1.7) (drill 1) (layers "*.Cu" "*.Mask" "B.SilkS") (remove_unused_layers no)
   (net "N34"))
  (pad "4" thru_hole circle (at -12.065 11.43 180) (size 1.7 1.7) (drill 1) (layers "*.Cu" "*.Mask" "B.SilkS") (remove_unused_layers no)
   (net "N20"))
  (pad "5" thru_hole circle (at -12.065 8.89 180) (size 1.7 1.7) (drill 1) (layers "*.Cu" "*.Mask" "B.SilkS") (remove_unused_layers no)
   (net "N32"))
  (pad "6" thru_hole circle (at -12.065 6.35 180) (size 1.7 1.7) (drill 1) (layers "*.Cu" "*.Mask" "B.SilkS") (remove_unused_layers no)
   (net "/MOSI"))
  (pad "7" thru_hole circle (at -12.065 3.81 180) (size 1.7 1.7) (drill 1) (layers "*.Cu" "*.Mask" "B.SilkS") (remove_unused_layers no)
   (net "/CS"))
  (pad "8" thru_hole circle (at -12.065 1.27 180) (size 1.7 1.7) (drill 1) (layers "*.Cu" "*.Mask" "B.SilkS") (remove_unused_layers no)
   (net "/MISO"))
  (pad "9" thru_hole circle (at -12.065 -1.27 180) (size 1.7 1.7) (drill 1) (layers "*.Cu" "*.Mask" "B.SilkS") (remove_unused_layers no)
   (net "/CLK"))
  (pad "10" thru_hole circle (at -12.065 -3.81 180) (size 1.7 1.7) (drill 1) (layers "*.Cu" "*.Mask" "B.SilkS") (remove_unused_layers no)
   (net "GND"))
  (pad "11" thru_hole circle (at -12.065 -6.35 180) (size 1.7 1.7) (drill 1) (layers "*.Cu" "*.Mask" "B.SilkS") (remove_unused_layers no)
   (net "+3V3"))
  (pad "12" thru_hole circle (at -12.065 -8.89 180) (size 1.7 1.7) (drill 1) (layers "*.Cu" "*.Mask" "B.SilkS") (remove_unused_layers no)
   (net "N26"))
  (pad "13" thru_hole circle (at -12.065 -11.43 180) (size 1.7 1.7) (drill 1) (layers "*.Cu" "*.Mask" "B.SilkS") (remove_unused_layers no)
   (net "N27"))
  (pad "14" thru_hole circle (at -12.065 -13.97 180) (size 1.7 1.7) (drill 1) (layers "*.Cu" "*.Mask" "B.SilkS") (remove_unused_layers no)
   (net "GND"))
  (pad "15" thru_hole circle (at -12.065 -16.51 180) (size 1.7 1.7) (drill 1) (layers "*.Cu" "*.Mask" "B.SilkS") (remove_unused_layers no)
   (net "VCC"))
  (pad "16" thru_hole circle (at 11.43 -16.51 180) (size 1.7 1.7) (drill 1) (layers "*.Cu" "*.Mask" "B.SilkS") (remove_unused_layers no)
   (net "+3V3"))
  (pad "17" thru_hole circle (at 11.43 -13.97 180) (size 1.7 1.7) (drill 1) (layers "*.Cu" "*.Mask" "B.SilkS") (remove_unused_layers no)
   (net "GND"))
  (pad "18" thru_hole circle (at 11.43 -11.43 180) (size 1.7 1.7) (drill 1) (layers "*.Cu" "*.Mask" "B.SilkS") (remove_unused_layers no)
   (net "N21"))
  (pad "19" thru_hole circle (at 11.43 -8.89 180) (size 1.7 1.7) (drill 1) (layers "*.Cu" "*.Mask" "B.SilkS") (remove_unused_layers no)
   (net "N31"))
  (pad "20" thru_hole circle (at 11.43 -6.35 180) (size 1.7 1.7) (drill 1) (layers "*.Cu" "*.Mask" "B.SilkS") (remove_unused_layers no)
   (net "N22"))
  (pad "21" thru_hole circle (at 11.43 -3.81 180) (size 1.7 1.7) (drill 1) (layers "*.Cu" "*.Mask" "B.SilkS") (remove_unused_layers no)
   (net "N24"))
  (pad "22" thru_hole circle (at 11.43 -1.27 180) (size 1.7 1.7) (drill 1) (layers "*.Cu" "*.Mask" "B.SilkS") (remove_unused_layers no)
   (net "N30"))
  (pad "23" thru_hole circle (at 11.43 1.27 180) (size 1.7 1.7) (drill 1) (layers "*.Cu" "*.Mask" "B.SilkS") (remove_unused_layers no)
   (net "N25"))
  (pad "24" thru_hole circle (at 11.43 3.81 180) (size 1.7 1.7) (drill 1) (layers "*.Cu" "*.Mask" "B.SilkS") (remove_unused_layers no)
   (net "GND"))
  (pad "25" thru_hole circle (at 11.43 6.35 180) (size 1.7 1.7) (drill 1) (layers "*.Cu" "*.Mask" "B.SilkS") (remove_unused_layers no)
   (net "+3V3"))
  (pad "26" thru_hole circle (at 11.43 8.89 180) (size 1.7 1.7) (drill 1) (layers "*.Cu" "*.Mask" "B.SilkS") (remove_unused_layers no)
   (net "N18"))
  (pad "27" thru_hole circle (at 11.43 11.43 180) (size 1.7 1.7) (drill 1) (layers "*.Cu" "*.Mask" "B.SilkS") (remove_unused_layers no)
   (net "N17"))
  (pad "28" thru_hole circle (at 11.43 13.97 180) (size 1.7 1.7) (drill 1) (layers "*.Cu" "*.Mask" "B.SilkS") (remove_unused_layers no)
   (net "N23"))
  (pad "29" thru_hole circle (at 11.43 16.51 180) (size 1.7 1.7) (drill 1) (layers "*.Cu" "*.Mask" "B.SilkS") (remove_unused_layers no)
   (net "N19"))
  (pad "30" thru_hole circle (at 11.43 19.05 180) (size 1.7 1.7) (drill 1) (layers "*.Cu" "*.Mask" "B.SilkS") (remove_unused_layers no)
   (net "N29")))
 (gr_rect (start 118.78 60.544) (end 147.25 104.092) (stroke (width 0.2) (type solid)) (fill no) (layer "Edge.Cuts"))
 (segment (start 127 70.6) (end 128 69.6) (width 0.254) (layer "F.Cu") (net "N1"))
 (segment (start 127 92.094) (end 127 70.6) (width 0.254) (layer "F.Cu") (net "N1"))
 (segment (start 128.096 93.19) (end 127 92.094) (width 0.254) (layer "F.Cu") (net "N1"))
 (segment (start 139.006 88.28) (end 144.6 88.28) (width 0.254) (layer "F.Cu") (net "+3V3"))
 (segment (start 134.096 93.19) (end 139.006 88.28) (width 0.254) (layer "F.Cu") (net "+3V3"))
 (segment (start 119.6 96.935) (end 121.105 98.44) (width 0.254) (layer "F.Cu") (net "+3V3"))
 (segment (start 121.105 75.58) (end 119.6 77.085) (width 0.254) (layer "F.Cu") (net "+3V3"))
 (segment (start 119.6 77.085) (end 119.6 96.935) (width 0.254) (layer "F.Cu") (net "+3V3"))
 (segment (start 140.2 73.8) (end 140.2 83.88) (width 0.254) (layer "B.Cu") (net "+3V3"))
 (segment (start 128 68.1) (end 121.105 74.995) (width 0.254) (layer "B.Cu") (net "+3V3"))
 (segment (start 121.105 74.995) (end 121.105 75.58) (width 0.254) (layer "B.Cu") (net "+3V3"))
 (segment (start 140.2 73.8) (end 133.7 73.8) (width 0.254) (layer "B.Cu") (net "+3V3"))
 (segment (start 133.7 73.8) (end 128 68.1) (width 0.254) (layer "B.Cu") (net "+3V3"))
 (segment (start 140.2 83.88) (end 144.6 88.28) (width 0.254) (layer "B.Cu") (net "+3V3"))
 (segment (start 122.235 76.99) (end 126.096 76.99) (width 0.254) (layer "F.Cu") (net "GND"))
 (segment (start 142.35 95.9) (end 144.6 95.9) (width 0.254) (layer "F.Cu") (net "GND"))
 (segment (start 121.105 78.12) (end 122.235 76.99) (width 0.254) (layer "F.Cu") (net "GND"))
 (segment (start 136.8125 101.4375) (end 137.6 100.65) (width 0.254) (layer "F.Cu") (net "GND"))
 (segment (start 145.087944 76.942) (end 146.6 78.454056) (width 0.254) (layer "F.Cu") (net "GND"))
 (segment (start 132.45 101.4375) (end 136.8125 101.4375) (width 0.254) (layer "F.Cu") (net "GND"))
 (segment (start 123.95 101.4375) (end 123.95 98.745) (width 0.254) (layer "F.Cu") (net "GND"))
 (segment (start 123.95 98.745) (end 121.105 95.9) (width 0.254) (layer "F.Cu") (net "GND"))
 (segment (start 146.6 83.74) (end 144.6 85.74) (width 0.254) (layer "F.Cu") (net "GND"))
 (segment (start 137.6 100.65) (end 142.35 95.9) (width 0.254) (layer "F.Cu") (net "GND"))
 (segment (start 140.096 76.99) (end 140.144 76.942) (width 0.254) (layer "F.Cu") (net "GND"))
 (segment (start 140.144 76.942) (end 145.087944 76.942) (width 0.254) (layer "F.Cu") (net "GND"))
 (segment (start 146.6 78.454056) (end 146.6 83.74) (width 0.254) (layer "F.Cu") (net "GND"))
 (segment (start 122.283 79.298) (end 122.283 94.722) (width 0.254) (layer "B.Cu") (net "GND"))
 (segment (start 145.778 94.722) (end 144.6 95.9) (width 0.254) (layer "B.Cu") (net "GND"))
 (segment (start 144.6 85.74) (end 145.778 86.918) (width 0.254) (layer "B.Cu") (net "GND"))
 (segment (start 123.95 98.745) (end 121.105 95.9) (width 0.254) (layer "B.Cu") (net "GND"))
 (segment (start 136.8125 101.4375) (end 137.6 100.65) (width 0.254) (layer "B.Cu") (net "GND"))
 (segment (start 121.105 78.12) (end 122.283 79.298) (width 0.254) (layer "B.Cu") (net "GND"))
 (segment (start 145.778 86.918) (end 145.778 94.722) (width 0.254) (layer "B.Cu") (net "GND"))
 (segment (start 132.45 101.4375) (end 136.8125 101.4375) (width 0.254) (layer "B.Cu") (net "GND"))
 (segment (start 123.95 101.4375) (end 123.95 98.745) (width 0.254) (layer "B.Cu") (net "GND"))
 (segment (start 122.283 94.722) (end 121.105 95.9) (width 0.254) (layer "B.Cu") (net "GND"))
 (segment (start 142.39 100.65) (end 144.6 98.44) (width 0.254) (layer "F.Cu") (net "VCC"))
 (segment (start 139.6 100.65) (end 142.39 100.65) (width 0.254) (layer "F.Cu") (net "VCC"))
 (segment (start 128.2 95.294) (end 126.096 93.19) (width 0.254) (layer "F.Cu") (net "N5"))
 (segment (start 128.2 101.4375) (end 128.2 95.294) (width 0.254) (layer "F.Cu") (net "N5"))
 (segment (start 144.6 80.66) (end 141.71 80.66) (width 0.254) (layer "F.Cu") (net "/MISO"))
 (segment (start 138.096 77.046) (end 138.096 76.99) (width 0.254) (layer "F.Cu") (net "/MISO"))
 (segment (start 141.71 80.66) (end 138.096 77.046) (width 0.254) (layer "F.Cu") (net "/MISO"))
 (segment (start 134.096 77.046) (end 134.096 76.99) (width 0.254) (layer "F.Cu") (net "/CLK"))
 (segment (start 144.6 83.2) (end 140.25 83.2) (width 0.254) (layer "F.Cu") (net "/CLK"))
 (segment (start 140.25 83.2) (end 134.096 77.046) (width 0.254) (layer "F.Cu") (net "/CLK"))
 (segment (start 144.6 78.12) (end 146 79.52) (width 0.254) (layer "F.Cu") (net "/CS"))
 (segment (start 146 79.52) (end 146 83.6) (width 0.254) (layer "F.Cu") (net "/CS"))
 (segment (start 139.668 84.562) (end 132.096 76.99) (width 0.254) (layer "F.Cu") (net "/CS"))
 (segment (start 145.038 84.562) (end 139.668 84.562) (width 0.254) (layer "F.Cu") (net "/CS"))
 (segment (start 146 83.6) (end 145.038 84.562) (width 0.254) (layer "F.Cu") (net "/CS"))
 (segment (start 136.096 76.99) (end 136.096 76.39) (width 0.254) (layer "F.Cu") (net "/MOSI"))
 (segment (start 136.906 75.58) (end 144.6 75.58) (width 0.254) (layer "F.Cu") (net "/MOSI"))
 (segment (start 136.096 76.39) (end 136.906 75.58) (width 0.254) (layer "F.Cu") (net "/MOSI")))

